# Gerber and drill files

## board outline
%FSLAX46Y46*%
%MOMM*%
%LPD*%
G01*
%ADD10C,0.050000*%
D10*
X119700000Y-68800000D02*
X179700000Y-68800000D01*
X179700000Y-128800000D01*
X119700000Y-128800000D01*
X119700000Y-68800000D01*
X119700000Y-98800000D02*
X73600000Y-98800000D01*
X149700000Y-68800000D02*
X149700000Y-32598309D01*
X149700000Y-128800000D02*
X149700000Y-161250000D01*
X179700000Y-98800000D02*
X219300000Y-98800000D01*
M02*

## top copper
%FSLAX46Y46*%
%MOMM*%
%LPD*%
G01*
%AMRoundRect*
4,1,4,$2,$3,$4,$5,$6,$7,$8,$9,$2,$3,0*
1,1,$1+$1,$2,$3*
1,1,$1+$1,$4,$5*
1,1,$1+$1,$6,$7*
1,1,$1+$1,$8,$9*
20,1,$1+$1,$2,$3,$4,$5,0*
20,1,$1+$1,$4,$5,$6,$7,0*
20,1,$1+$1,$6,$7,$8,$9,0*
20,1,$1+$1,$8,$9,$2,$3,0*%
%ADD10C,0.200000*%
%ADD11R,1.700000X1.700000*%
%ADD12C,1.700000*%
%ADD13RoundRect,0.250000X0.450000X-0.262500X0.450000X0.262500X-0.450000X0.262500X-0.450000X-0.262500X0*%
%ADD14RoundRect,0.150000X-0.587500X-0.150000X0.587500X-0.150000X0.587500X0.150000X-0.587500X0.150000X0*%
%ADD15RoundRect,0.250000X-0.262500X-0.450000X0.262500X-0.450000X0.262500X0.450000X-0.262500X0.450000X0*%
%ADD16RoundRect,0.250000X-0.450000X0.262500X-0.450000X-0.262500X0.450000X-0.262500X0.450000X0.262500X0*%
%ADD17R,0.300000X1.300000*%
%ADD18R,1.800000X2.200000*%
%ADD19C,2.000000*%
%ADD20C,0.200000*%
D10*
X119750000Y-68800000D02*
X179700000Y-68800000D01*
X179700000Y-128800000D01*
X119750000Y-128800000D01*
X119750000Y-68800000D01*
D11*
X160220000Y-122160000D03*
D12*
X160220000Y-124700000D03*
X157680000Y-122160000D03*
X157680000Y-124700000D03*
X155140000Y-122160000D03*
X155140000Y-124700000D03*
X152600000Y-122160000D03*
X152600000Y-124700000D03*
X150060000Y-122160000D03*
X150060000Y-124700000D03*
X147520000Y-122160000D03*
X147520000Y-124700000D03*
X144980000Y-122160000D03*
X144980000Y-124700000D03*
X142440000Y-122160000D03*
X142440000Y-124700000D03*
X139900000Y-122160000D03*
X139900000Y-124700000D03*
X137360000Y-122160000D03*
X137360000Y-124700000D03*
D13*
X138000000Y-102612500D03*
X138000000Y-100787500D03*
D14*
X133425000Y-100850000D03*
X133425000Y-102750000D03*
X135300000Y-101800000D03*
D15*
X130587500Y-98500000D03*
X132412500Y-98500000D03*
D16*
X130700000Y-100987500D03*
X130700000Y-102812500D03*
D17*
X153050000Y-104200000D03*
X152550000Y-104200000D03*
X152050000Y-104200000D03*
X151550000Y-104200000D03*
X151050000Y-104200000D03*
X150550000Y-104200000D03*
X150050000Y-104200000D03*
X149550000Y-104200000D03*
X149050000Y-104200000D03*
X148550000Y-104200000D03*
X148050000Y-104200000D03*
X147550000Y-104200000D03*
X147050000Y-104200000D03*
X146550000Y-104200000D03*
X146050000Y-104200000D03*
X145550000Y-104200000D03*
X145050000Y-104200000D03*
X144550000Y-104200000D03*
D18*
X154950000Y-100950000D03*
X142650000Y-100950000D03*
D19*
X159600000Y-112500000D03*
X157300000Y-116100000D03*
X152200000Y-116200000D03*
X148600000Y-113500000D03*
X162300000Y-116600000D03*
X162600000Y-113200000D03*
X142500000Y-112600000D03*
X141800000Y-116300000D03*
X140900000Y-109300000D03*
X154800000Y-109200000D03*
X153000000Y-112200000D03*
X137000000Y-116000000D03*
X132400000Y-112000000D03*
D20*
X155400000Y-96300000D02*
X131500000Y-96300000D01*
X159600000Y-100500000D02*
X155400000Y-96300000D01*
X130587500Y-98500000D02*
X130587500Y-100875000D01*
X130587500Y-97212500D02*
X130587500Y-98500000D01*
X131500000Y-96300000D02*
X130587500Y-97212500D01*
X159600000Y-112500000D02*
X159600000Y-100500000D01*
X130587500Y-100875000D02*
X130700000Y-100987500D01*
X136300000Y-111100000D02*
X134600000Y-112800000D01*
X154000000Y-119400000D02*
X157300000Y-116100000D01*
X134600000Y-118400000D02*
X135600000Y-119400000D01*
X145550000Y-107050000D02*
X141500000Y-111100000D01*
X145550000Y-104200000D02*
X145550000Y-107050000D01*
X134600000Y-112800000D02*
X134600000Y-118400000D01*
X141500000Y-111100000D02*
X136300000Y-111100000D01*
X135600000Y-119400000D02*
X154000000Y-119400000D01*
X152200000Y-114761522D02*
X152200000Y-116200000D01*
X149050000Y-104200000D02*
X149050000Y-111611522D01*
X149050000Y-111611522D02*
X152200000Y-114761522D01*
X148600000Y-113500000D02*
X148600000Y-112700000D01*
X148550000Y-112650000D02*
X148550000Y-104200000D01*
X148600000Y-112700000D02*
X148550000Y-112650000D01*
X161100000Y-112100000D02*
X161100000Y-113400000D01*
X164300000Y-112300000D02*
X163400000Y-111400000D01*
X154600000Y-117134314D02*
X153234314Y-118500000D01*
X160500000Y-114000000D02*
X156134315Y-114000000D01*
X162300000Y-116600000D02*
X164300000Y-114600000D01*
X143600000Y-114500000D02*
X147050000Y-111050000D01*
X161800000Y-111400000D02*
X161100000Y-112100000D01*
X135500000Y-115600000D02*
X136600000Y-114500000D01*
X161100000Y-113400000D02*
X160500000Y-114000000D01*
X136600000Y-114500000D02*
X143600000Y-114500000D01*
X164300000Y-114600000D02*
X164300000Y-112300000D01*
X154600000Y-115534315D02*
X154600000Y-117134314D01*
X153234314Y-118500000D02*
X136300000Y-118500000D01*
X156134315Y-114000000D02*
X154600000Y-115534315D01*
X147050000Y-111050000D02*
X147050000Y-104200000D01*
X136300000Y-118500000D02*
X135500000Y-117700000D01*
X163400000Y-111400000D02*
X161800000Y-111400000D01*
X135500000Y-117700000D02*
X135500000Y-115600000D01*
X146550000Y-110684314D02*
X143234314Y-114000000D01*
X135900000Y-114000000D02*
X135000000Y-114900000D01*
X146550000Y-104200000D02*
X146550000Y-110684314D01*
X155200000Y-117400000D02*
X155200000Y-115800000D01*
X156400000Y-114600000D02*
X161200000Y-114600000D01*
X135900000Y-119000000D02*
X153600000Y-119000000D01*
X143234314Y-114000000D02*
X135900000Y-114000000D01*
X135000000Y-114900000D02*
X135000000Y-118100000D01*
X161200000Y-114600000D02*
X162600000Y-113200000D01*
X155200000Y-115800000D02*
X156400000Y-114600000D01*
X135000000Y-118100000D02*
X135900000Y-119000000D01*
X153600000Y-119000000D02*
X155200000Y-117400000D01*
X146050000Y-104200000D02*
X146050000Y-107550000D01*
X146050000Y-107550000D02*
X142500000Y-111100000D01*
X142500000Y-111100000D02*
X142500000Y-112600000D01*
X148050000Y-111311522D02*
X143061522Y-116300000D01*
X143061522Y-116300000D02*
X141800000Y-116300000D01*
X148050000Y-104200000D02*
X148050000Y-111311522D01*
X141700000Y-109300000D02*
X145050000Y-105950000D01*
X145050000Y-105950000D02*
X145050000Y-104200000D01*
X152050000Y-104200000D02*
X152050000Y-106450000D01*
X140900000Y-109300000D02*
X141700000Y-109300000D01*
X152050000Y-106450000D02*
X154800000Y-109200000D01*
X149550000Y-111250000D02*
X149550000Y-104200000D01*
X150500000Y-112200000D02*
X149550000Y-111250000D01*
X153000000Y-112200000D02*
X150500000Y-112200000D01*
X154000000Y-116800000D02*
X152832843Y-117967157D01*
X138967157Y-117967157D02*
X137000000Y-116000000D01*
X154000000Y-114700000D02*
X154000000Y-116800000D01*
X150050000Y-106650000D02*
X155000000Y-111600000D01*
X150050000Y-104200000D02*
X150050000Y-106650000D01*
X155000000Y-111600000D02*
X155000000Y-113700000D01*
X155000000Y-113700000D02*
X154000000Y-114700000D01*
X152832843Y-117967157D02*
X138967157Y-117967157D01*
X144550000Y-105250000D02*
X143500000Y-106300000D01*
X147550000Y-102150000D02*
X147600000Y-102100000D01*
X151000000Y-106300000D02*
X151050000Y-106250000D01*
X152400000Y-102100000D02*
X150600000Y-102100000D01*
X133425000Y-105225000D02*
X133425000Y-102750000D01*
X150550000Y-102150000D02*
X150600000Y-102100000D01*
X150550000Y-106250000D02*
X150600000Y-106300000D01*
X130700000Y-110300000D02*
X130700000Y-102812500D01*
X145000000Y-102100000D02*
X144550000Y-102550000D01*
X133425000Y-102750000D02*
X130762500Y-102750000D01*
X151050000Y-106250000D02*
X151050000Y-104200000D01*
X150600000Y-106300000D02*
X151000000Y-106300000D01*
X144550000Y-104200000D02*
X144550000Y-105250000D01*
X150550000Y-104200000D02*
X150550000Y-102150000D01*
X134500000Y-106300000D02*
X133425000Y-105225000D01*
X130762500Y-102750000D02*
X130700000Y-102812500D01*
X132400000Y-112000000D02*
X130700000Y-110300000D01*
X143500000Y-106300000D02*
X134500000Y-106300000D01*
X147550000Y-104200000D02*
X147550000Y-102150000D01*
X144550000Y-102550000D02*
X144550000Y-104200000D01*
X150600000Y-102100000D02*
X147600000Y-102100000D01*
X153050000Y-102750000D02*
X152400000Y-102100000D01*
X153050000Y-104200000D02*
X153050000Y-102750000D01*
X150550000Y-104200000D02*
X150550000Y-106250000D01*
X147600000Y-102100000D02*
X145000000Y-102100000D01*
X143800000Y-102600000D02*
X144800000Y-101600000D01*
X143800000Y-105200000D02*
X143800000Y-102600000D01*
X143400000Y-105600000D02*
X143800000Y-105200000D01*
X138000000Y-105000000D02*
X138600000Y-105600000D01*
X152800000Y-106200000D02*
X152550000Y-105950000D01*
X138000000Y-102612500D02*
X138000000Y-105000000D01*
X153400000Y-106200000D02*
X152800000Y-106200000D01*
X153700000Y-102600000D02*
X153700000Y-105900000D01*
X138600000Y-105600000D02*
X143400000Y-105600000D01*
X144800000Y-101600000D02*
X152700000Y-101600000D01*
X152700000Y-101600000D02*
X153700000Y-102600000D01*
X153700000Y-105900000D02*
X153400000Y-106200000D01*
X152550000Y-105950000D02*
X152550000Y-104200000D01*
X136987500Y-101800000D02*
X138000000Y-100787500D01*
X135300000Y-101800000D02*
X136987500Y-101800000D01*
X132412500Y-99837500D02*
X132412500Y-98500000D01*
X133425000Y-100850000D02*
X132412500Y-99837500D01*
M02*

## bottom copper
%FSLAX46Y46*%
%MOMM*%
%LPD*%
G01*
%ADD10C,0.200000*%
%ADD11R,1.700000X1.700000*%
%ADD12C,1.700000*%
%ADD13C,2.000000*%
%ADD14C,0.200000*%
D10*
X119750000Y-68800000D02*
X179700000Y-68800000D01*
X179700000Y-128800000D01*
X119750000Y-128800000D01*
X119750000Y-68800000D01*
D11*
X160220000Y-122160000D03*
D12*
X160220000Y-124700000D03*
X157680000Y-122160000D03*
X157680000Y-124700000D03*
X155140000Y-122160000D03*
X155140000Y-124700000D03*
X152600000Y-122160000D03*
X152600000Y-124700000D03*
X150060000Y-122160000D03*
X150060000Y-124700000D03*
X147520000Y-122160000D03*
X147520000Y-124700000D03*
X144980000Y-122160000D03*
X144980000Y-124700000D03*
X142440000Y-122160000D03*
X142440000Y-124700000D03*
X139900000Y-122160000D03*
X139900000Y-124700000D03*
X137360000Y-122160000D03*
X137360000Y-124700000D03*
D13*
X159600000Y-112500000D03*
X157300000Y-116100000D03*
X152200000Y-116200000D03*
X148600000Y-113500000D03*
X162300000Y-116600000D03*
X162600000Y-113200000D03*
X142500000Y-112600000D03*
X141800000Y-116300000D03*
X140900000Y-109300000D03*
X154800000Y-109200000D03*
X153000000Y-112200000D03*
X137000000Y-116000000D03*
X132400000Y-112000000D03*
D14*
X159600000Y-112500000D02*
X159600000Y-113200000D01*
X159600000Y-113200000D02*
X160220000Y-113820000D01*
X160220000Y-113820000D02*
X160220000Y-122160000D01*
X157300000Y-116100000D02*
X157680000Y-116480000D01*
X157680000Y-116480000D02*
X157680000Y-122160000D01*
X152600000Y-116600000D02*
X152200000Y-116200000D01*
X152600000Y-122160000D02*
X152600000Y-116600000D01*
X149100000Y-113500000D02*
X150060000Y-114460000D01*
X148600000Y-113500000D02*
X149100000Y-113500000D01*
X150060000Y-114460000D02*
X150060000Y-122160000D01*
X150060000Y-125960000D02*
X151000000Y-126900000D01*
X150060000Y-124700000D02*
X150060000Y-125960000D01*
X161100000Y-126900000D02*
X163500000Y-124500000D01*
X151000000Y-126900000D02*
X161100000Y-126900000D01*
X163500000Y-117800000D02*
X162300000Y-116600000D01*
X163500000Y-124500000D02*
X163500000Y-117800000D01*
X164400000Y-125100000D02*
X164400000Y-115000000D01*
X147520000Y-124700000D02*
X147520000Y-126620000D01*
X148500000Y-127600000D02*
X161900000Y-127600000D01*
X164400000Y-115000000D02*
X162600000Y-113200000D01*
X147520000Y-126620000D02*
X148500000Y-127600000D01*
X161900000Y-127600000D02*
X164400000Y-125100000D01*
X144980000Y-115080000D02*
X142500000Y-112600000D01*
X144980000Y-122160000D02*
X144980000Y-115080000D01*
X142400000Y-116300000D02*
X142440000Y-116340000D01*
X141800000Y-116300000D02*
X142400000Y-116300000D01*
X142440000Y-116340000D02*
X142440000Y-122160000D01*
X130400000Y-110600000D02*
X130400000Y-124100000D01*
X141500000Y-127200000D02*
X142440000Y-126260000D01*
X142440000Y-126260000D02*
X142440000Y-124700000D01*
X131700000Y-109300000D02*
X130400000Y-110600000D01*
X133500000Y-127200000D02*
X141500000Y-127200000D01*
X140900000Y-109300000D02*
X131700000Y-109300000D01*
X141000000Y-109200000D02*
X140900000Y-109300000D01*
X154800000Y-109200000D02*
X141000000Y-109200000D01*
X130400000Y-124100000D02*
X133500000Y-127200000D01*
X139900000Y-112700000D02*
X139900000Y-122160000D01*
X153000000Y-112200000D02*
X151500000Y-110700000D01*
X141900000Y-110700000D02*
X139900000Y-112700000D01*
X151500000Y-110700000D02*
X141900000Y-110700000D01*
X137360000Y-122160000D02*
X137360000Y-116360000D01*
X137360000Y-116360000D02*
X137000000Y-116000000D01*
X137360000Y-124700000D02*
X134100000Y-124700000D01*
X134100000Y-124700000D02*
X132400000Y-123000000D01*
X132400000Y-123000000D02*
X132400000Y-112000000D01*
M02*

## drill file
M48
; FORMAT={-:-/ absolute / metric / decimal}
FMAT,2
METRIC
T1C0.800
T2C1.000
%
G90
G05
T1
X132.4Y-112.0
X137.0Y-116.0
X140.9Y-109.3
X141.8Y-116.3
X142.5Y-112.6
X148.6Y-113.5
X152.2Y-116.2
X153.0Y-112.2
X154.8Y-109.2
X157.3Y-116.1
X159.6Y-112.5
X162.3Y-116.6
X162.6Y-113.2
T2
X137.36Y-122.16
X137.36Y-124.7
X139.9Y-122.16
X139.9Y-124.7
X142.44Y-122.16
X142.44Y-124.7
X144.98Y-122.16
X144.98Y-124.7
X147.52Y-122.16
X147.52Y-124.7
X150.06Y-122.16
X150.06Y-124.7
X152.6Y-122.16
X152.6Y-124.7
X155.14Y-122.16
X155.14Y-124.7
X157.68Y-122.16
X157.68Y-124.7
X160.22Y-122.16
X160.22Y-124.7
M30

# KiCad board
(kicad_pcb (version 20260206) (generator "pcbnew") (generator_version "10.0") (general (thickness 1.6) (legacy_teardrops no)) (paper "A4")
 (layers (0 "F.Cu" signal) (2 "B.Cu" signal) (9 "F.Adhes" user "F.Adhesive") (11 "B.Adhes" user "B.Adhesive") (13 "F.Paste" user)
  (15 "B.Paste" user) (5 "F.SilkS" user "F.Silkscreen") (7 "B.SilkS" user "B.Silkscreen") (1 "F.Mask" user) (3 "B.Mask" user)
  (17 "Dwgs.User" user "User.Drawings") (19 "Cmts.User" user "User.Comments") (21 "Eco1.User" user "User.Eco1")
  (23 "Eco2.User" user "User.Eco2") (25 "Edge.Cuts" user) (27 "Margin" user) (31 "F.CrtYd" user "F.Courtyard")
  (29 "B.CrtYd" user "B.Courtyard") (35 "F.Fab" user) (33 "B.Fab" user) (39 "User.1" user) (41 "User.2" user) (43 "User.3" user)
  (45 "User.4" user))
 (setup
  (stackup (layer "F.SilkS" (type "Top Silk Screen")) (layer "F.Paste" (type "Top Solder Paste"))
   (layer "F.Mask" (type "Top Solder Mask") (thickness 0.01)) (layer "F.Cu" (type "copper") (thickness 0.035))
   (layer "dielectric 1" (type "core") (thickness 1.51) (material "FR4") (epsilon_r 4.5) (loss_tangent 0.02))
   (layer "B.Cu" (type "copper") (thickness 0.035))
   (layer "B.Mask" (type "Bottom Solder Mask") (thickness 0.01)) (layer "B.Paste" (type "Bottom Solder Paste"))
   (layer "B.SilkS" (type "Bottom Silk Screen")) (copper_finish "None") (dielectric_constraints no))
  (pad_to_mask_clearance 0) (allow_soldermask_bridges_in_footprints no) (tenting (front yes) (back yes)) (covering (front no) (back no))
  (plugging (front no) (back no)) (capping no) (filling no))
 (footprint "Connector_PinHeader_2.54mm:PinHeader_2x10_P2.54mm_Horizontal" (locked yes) (layer "F.Cu") (at 160.22 122.16 -90)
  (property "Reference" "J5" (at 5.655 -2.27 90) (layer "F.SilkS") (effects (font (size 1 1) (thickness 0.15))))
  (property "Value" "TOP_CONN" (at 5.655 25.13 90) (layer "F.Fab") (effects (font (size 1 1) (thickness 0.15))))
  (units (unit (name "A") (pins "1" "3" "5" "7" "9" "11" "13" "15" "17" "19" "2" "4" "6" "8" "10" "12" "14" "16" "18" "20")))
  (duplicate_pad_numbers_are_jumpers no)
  (pad "1" thru_hole rect (at 0 0 270) (size 1.7 1.7) (drill 1) (layers "*.Cu" "*.Mask") (remove_unused_layers no) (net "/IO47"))
  (pad "2" thru_hole circle (at 2.54 0 270) (size 1.7 1.7) (drill 1) (layers "*.Cu" "*.Mask") (remove_unused_layers no) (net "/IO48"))
  (pad "3" thru_hole circle (at 0 2.54 270) (size 1.7 1.7) (drill 1) (layers "*.Cu" "*.Mask") (remove_unused_layers no) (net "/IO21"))
  (pad "4" thru_hole circle (at 2.54 2.54 270) (size 1.7 1.7) (drill 1) (layers "*.Cu" "*.Mask") (remove_unused_layers no) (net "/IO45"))
  (pad "5" thru_hole circle (at 0 5.08 270) (size 1.7 1.7) (drill 1) (layers "*.Cu" "*.Mask") (remove_unused_layers no) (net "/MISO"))
  (pad "6" thru_hole circle (at 2.54 5.08 270) (size 1.7 1.7) (drill 1) (layers "*.Cu" "*.Mask") (remove_unused_layers no) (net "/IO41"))
  (pad "7" thru_hole circle (at 0 7.62 270) (size 1.7 1.7) (drill 1) (layers "*.Cu" "*.Mask") (remove_unused_layers no) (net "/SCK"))
  (pad "8" thru_hole circle (at 2.54 7.62 270) (size 1.7 1.7) (drill 1) (layers "*.Cu" "*.Mask") (remove_unused_layers no) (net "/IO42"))
  (pad "9" thru_hole circle (at 0 10.16 270) (size 1.7 1.7) (drill 1) (layers "*.Cu" "*.Mask") (remove_unused_layers no) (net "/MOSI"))
  (pad "10" thru_hole circle (at 2.54 10.16 270) (size 1.7 1.7) (drill 1) (layers "*.Cu" "*.Mask") (remove_unused_layers no) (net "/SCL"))
  (pad "11" thru_hole circle (at 0 12.7 270) (size 1.7 1.7) (drill 1) (layers "*.Cu" "*.Mask") (remove_unused_layers no) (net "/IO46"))
  (pad "12" thru_hole circle (at 2.54 12.7 270) (size 1.7 1.7) (drill 1) (layers "*.Cu" "*.Mask") (remove_unused_layers no) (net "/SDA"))
  (pad "13" thru_hole circle (at 0 15.24 270) (size 1.7 1.7) (drill 1) (layers "*.Cu" "*.Mask") (remove_unused_layers no) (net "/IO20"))
  (pad "14" thru_hole circle (at 2.54 15.24 270) (size 1.7 1.7) (drill 1) (layers "*.Cu" "*.Mask") (remove_unused_layers no) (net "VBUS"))
  (pad "15" thru_hole circle (at 0 17.78 270) (size 1.7 1.7) (drill 1) (layers "*.Cu" "*.Mask") (remove_unused_layers no) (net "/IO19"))
  (pad "16" thru_hole circle (at 2.54 17.78 270) (size 1.7 1.7) (drill 1) (layers "*.Cu" "*.Mask") (remove_unused_layers no) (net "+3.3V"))
  (pad "17" thru_hole circle (at 0 20.32 270) (size 1.7 1.7) (drill 1) (layers "*.Cu" "*.Mask") (remove_unused_layers no) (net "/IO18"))
  (pad "18" thru_hole circle (at 2.54 20.32 270) (size 1.7 1.7) (drill 1) (layers "*.Cu" "*.Mask") (remove_unused_layers no) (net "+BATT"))
  (pad "19" thru_hole circle (at 0 22.86 270) (size 1.7 1.7) (drill 1) (layers "*.Cu" "*.Mask") (remove_unused_layers no) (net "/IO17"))
  (pad "20" thru_hole circle (at 2.54 22.86 270) (size 1.7 1.7) (drill 1) (layers "*.Cu" "*.Mask") (remove_unused_layers no) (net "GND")))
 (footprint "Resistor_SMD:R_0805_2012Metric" (layer "F.Cu") (at 138 101.7 90)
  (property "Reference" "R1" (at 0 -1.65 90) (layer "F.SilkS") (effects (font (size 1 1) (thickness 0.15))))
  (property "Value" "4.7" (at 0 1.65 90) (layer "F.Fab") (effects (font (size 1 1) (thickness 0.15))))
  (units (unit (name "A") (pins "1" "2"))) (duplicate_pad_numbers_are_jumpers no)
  (pad "1" smd roundrect (at -0.9125 0 90) (size 1.025 1.4) (layers "F.Cu" "F.Mask" "F.Paste") (roundrect_rratio 0.243902) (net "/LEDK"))
  (pad "2" smd roundrect (at 0.9125 0 90) (size 1.025 1.4) (layers "F.Cu" "F.Mask" "F.Paste") (roundrect_rratio 0.243902) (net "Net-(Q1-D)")))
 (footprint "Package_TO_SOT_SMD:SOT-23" (layer "F.Cu") (at 134.3625 101.8)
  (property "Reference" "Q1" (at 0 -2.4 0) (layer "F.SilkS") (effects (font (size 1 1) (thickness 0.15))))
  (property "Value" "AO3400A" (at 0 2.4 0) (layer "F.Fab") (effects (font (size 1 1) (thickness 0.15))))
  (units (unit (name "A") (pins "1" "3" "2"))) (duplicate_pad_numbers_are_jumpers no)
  (pad "1" smd roundrect (at -0.9375 -0.95) (size 1.475 0.6) (layers "F.Cu" "F.Mask" "F.Paste") (roundrect_rratio 0.25) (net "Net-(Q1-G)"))
  (pad "2" smd roundrect (at -0.9375 0.95) (size 1.475 0.6) (layers "F.Cu" "F.Mask" "F.Paste") (roundrect_rratio 0.25) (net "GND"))
  (pad "3" smd roundrect (at 0.9375 0) (size 1.475 0.6) (layers "F.Cu" "F.Mask" "F.Paste") (roundrect_rratio 0.25) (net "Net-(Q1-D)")))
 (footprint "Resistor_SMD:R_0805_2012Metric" (layer "F.Cu") (at 131.5 98.5)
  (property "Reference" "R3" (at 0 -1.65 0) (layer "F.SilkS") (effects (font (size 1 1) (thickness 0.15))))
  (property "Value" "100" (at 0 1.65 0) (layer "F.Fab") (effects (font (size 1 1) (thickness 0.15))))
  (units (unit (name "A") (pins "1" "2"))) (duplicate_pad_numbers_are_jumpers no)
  (pad "1" smd roundrect (at -0.9125 0) (size 1.025 1.4) (layers "F.Cu" "F.Mask" "F.Paste") (roundrect_rratio 0.243902) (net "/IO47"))
  (pad "2" smd roundrect (at 0.9125 0) (size 1.025 1.4) (layers "F.Cu" "F.Mask" "F.Paste") (roundrect_rratio 0.243902) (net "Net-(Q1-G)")))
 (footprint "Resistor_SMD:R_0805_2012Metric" (layer "F.Cu") (at 130.7 101.9 -90)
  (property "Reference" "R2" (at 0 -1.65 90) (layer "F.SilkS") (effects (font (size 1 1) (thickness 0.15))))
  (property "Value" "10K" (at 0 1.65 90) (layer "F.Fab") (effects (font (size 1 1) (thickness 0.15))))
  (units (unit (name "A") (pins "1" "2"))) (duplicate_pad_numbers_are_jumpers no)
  (pad "1" smd roundrect (at -0.9125 0 270) (size 1.025 1.4) (layers "F.Cu" "F.Mask" "F.Paste") (roundrect_rratio 0.243902) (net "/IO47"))
  (pad "2" smd roundrect (at 0.9125 0 270) (size 1.025 1.4) (layers "F.Cu" "F.Mask" "F.Paste") (roundrect_rratio 0.243902) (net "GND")))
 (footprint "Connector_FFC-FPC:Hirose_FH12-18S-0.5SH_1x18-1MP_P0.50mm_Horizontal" (layer "F.Cu") (at 148.8 102.35 180)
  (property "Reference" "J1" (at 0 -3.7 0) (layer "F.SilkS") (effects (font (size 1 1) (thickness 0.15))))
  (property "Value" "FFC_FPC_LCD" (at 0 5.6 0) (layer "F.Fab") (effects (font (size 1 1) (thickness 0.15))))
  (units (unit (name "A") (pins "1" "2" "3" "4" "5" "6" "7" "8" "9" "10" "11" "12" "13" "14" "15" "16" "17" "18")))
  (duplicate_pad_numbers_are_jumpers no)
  (pad "1" smd rect (at -4.25 -1.85 180) (size 0.3 1.3) (layers "F.Cu" "F.Mask" "F.Paste") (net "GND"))
  (pad "2" smd rect (at -3.75 -1.85 180) (size 0.3 1.3) (layers "F.Cu" "F.Mask" "F.Paste") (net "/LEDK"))
  (pad "3" smd rect (at -3.25 -1.85 180) (size 0.3 1.3) (layers "F.Cu" "F.Mask" "F.Paste") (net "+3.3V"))
  (pad "4" smd rect (at -2.75 -1.85 180) (size 0.3 1.3) (layers "F.Cu" "F.Mask" "F.Paste") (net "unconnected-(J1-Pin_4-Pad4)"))
  (pad "5" smd rect (at -2.25 -1.85 180) (size 0.3 1.3) (layers "F.Cu" "F.Mask" "F.Paste") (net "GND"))
  (pad "6" smd rect (at -1.75 -1.85 180) (size 0.3 1.3) (layers "F.Cu" "F.Mask" "F.Paste") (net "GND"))
  (pad "7" smd rect (at -1.25 -1.85 180) (size 0.3 1.3) (layers "F.Cu" "F.Mask" "F.Paste") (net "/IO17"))
  (pad "8" smd rect (at -0.75 -1.85 180) (size 0.3 1.3) (layers "F.Cu" "F.Mask" "F.Paste") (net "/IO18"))
  (pad "9" smd rect (at -0.25 -1.85 180) (size 0.3 1.3) (layers "F.Cu" "F.Mask" "F.Paste") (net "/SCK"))
  (pad "10" smd rect (at 0.25 -1.85 180) (size 0.3 1.3) (layers "F.Cu" "F.Mask" "F.Paste") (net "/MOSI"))
  (pad "11" smd rect (at 0.75 -1.85 180) (size 0.3 1.3) (layers "F.Cu" "F.Mask" "F.Paste") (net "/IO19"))
  (pad "12" smd rect (at 1.25 -1.85 180) (size 0.3 1.3) (layers "F.Cu" "F.Mask" "F.Paste") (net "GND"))
  (pad "13" smd rect (at 1.75 -1.85 180) (size 0.3 1.3) (layers "F.Cu" "F.Mask" "F.Paste") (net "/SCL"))
  (pad "14" smd rect (at 2.25 -1.85 180) (size 0.3 1.3) (layers "F.Cu" "F.Mask" "F.Paste") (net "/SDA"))
  (pad "15" smd rect (at 2.75 -1.85 180) (size 0.3 1.3) (layers "F.Cu" "F.Mask" "F.Paste") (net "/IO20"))
  (pad "16" smd rect (at 3.25 -1.85 180) (size 0.3 1.3) (layers "F.Cu" "F.Mask" "F.Paste") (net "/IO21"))
  (pad "17" smd rect (at 3.75 -1.85 180) (size 0.3 1.3) (layers "F.Cu" "F.Mask" "F.Paste") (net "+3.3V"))
  (pad "18" smd rect (at 4.25 -1.85 180) (size 0.3 1.3) (layers "F.Cu" "F.Mask" "F.Paste") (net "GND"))
  (pad "MP" smd rect (at -6.15 1.4 180) (size 1.8 2.2) (layers "F.Cu" "F.Mask" "F.Paste"))
  (pad "MP" smd rect (at 6.15 1.4 180) (size 1.8 2.2) (layers "F.Cu" "F.Mask" "F.Paste")))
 (gr_rect (start 119.75 68.8) (end 179.7 128.8) (stroke (width 0.2) (type default)) (fill no) (layer "F.Cu"))
 (gr_rect (start 119.75 68.8) (end 179.7 128.8) (stroke (width 0.2) (type default)) (fill no) (layer "B.Cu"))
 (gr_rect (start 119.7 68.8) (end 179.7 128.8) (stroke (width 0.05) (type solid)) (fill no) (layer "Edge.Cuts"))
 (gr_line (start 119.7 98.8) (end 73.6 98.8) (stroke (width 0.05) (type default)) (layer "Edge.Cuts"))
 (gr_line (start 149.7 68.8) (end 149.7 32.598309) (stroke (width 0.05) (type solid)) (layer "Edge.Cuts"))
 (gr_line (start 149.7 128.8) (end 149.7 161.25) (stroke (width 0.05) (type default)) (layer "Edge.Cuts"))
 (gr_line (start 179.7 98.8) (end 219.3 98.8) (stroke (width 0.05) (type default)) (layer "Edge.Cuts"))
 (segment (start 155.4 96.3) (end 131.5 96.3) (width 0.2) (layer "F.Cu") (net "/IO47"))
 (segment (start 159.6 100.5) (end 155.4 96.3) (width 0.2) (layer "F.Cu") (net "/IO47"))
 (segment (start 130.5875 98.5) (end 130.5875 100.875) (width 0.2) (layer "F.Cu") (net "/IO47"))
 (segment (start 130.5875 97.2125) (end 130.5875 98.5) (width 0.2) (layer "F.Cu") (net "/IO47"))
 (segment (start 131.5 96.3) (end 130.5875 97.2125) (width 0.2) (layer "F.Cu") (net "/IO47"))
 (segment (start 159.6 112.5) (end 159.6 100.5) (width 0.2) (layer "F.Cu") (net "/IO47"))
 (segment (start 130.5875 100.875) (end 130.7 100.9875) (width 0.2) (layer "F.Cu") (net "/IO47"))
 (via (at 159.6 112.5) (size 2) (drill 0.8) (layers "F.Cu" "B.Cu") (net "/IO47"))
 (segment (start 159.6 112.5) (end 159.6 113.2) (width 0.2) (layer "B.Cu") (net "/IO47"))
 (segment (start 159.6 113.2) (end 160.22 113.82) (width 0.2) (layer "B.Cu") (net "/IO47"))
 (segment (start 160.22 113.82) (end 160.22 122.16) (width 0.2) (layer "B.Cu") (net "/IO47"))
 (segment (start 136.3 111.1) (end 134.6 112.8) (width 0.2) (layer "F.Cu") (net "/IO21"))
 (segment (start 154 119.4) (end 157.3 116.1) (width 0.2) (layer "F.Cu") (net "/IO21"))
 (segment (start 134.6 118.4) (end 135.6 119.4) (width 0.2) (layer "F.Cu") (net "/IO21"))
 (segment (start 145.55 107.05) (end 141.5 111.1) (width 0.2) (layer "F.Cu") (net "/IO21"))
 (segment (start 145.55 104.2) (end 145.55 107.05) (width 0.2) (layer "F.Cu") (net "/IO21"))
 (segment (start 134.6 112.8) (end 134.6 118.4) (width 0.2) (layer "F.Cu") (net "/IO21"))
 (segment (start 141.5 111.1) (end 136.3 111.1) (width 0.2) (layer "F.Cu") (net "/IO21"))
 (segment (start 135.6 119.4) (end 154 119.4) (width 0.2) (layer "F.Cu") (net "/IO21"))
 (via (at 157.3 116.1) (size 2) (drill 0.8) (layers "F.Cu" "B.Cu") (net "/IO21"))
 (segment (start 157.3 116.1) (end 157.68 116.48) (width 0.2) (layer "B.Cu") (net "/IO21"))
 (segment (start 157.68 116.48) (end 157.68 122.16) (width 0.2) (layer "B.Cu") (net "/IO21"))
 (segment (start 152.2 114.761522) (end 152.2 116.2) (width 0.2) (layer "F.Cu") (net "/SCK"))
 (segment (start 149.05 104.2) (end 149.05 111.611522) (width 0.2) (layer "F.Cu") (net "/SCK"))
 (segment (start 149.05 111.611522) (end 152.2 114.761522) (width 0.2) (layer "F.Cu") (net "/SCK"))
 (via (at 152.2 116.2) (size 2) (drill 0.8) (layers "F.Cu" "B.Cu") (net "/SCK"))
 (segment (start 152.6 116.6) (end 152.2 116.2) (width 0.2) (layer "B.Cu") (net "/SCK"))
 (segment (start 152.6 122.16) (end 152.6 116.6) (width 0.2) (layer "B.Cu") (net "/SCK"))
 (segment (start 148.6 113.5) (end 148.6 112.7) (width 0.2) (layer "F.Cu") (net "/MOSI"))
 (segment (start 148.55 112.65) (end 148.55 104.2) (width 0.2) (layer "F.Cu") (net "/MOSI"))
 (segment (start 148.6 112.7) (end 148.55 112.65) (width 0.2) (layer "F.Cu") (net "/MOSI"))
 (via (at 148.6 113.5) (size 2) (drill 0.8) (layers "F.Cu" "B.Cu") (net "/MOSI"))
 (segment (start 149.1 113.5) (end 150.06 114.46) (width 0.2) (layer "B.Cu") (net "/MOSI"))
 (segment (start 148.6 113.5) (end 149.1 113.5) (width 0.2) (layer "B.Cu") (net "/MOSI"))
 (segment (start 150.06 114.46) (end 150.06 122.16) (width 0.2) (layer "B.Cu") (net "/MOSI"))
 (segment (start 161.1 112.1) (end 161.1 113.4) (width 0.2) (layer "F.Cu") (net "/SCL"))
 (segment (start 164.3 112.3) (end 163.4 111.4) (width 0.2) (layer "F.Cu") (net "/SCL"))
 (segment (start 154.6 117.134314) (end 153.234314 118.5) (width 0.2) (layer "F.Cu") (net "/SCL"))
 (segment (start 160.5 114) (end 156.134315 114) (width 0.2) (layer "F.Cu") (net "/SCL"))
 (segment (start 162.3 116.6) (end 164.3 114.6) (width 0.2) (layer "F.Cu") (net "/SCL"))
 (segment (start 143.6 114.5) (end 147.05 111.05) (width 0.2) (layer "F.Cu") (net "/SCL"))
 (segment (start 161.8 111.4) (end 161.1 112.1) (width 0.2) (layer "F.Cu") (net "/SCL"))
 (segment (start 135.5 115.6) (end 136.6 114.5) (width 0.2) (layer "F.Cu") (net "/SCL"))
 (segment (start 161.1 113.4) (end 160.5 114) (width 0.2) (layer "F.Cu") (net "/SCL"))
 (segment (start 136.6 114.5) (end 143.6 114.5) (width 0.2) (layer "F.Cu") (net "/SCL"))
 (segment (start 164.3 114.6) (end 164.3 112.3) (width 0.2) (layer "F.Cu") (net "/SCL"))
 (segment (start 154.6 115.534315) (end 154.6 117.134314) (width 0.2) (layer "F.Cu") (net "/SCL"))
 (segment (start 153.234314 118.5) (end 136.3 118.5) (width 0.2) (layer "F.Cu") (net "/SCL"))
 (segment (start 156.134315 114) (end 154.6 115.534315) (width 0.2) (layer "F.Cu") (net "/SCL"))
 (segment (start 147.05 111.05) (end 147.05 104.2) (width 0.2) (layer "F.Cu") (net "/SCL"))
 (segment (start 136.3 118.5) (end 135.5 117.7) (width 0.2) (layer "F.Cu") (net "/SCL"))
 (segment (start 163.4 111.4) (end 161.8 111.4) (width 0.2) (layer "F.Cu") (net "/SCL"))
 (segment (start 135.5 117.7) (end 135.5 115.6) (width 0.2) (layer "F.Cu") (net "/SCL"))
 (via (at 162.3 116.6) (size 2) (drill 0.8) (layers "F.Cu" "B.Cu") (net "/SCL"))
 (segment (start 150.06 125.96) (end 151 126.9) (width 0.2) (layer "B.Cu") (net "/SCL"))
 (segment (start 150.06 124.7) (end 150.06 125.96) (width 0.2) (layer "B.Cu") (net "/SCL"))
 (segment (start 161.1 126.9) (end 163.5 124.5) (width 0.2) (layer "B.Cu") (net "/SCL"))
 (segment (start 151 126.9) (end 161.1 126.9) (width 0.2) (layer "B.Cu") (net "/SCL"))
 (segment (start 163.5 117.8) (end 162.3 116.6) (width 0.2) (layer "B.Cu") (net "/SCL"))
 (segment (start 163.5 124.5) (end 163.5 117.8) (width 0.2) (layer "B.Cu") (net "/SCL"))
 (segment (start 146.55 110.684314) (end 143.234314 114) (width 0.2) (layer "F.Cu") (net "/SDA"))
 (segment (start 135.9 114) (end 135 114.9) (width 0.2) (layer "F.Cu") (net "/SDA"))
 (segment (start 146.55 104.2) (end 146.55 110.684314) (width 0.2) (layer "F.Cu") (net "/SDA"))
 (segment (start 155.2 117.4) (end 155.2 115.8) (width 0.2) (layer "F.Cu") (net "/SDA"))
 (segment (start 156.4 114.6) (end 161.2 114.6) (width 0.2) (layer "F.Cu") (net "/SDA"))
 (segment (start 135.9 119) (end 153.6 119) (width 0.2) (layer "F.Cu") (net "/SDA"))
 (segment (start 143.234314 114) (end 135.9 114) (width 0.2) (layer "F.Cu") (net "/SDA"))
 (segment (start 135 114.9) (end 135 118.1) (width 0.2) (layer "F.Cu") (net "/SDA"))
 (segment (start 161.2 114.6) (end 162.6 113.2) (width 0.2) (layer "F.Cu") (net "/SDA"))
 (segment (start 155.2 115.8) (end 156.4 114.6) (width 0.2) (layer "F.Cu") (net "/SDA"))
 (segment (start 135 118.1) (end 135.9 119) (width 0.2) (layer "F.Cu") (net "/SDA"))
 (segment (start 153.6 119) (end 155.2 117.4) (width 0.2) (layer "F.Cu") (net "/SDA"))
 (via (at 162.6 113.2) (size 2) (drill 0.8) (layers "F.Cu" "B.Cu") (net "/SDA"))
 (segment (start 164.4 125.1) (end 164.4 115) (width 0.2) (layer "B.Cu") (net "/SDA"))
 (segment (start 147.52 124.7) (end 147.52 126.62) (width 0.2) (layer "B.Cu") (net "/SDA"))
 (segment (start 148.5 127.6) (end 161.9 127.6) (width 0.2) (layer "B.Cu") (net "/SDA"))
 (segment (start 164.4 115) (end 162.6 113.2) (width 0.2) (layer "B.Cu") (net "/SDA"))
 (segment (start 147.52 126.62) (end 148.5 127.6) (width 0.2) (layer "B.Cu") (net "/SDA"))
 (segment (start 161.9 127.6) (end 164.4 125.1) (width 0.2) (layer "B.Cu") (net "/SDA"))
 (segment (start 146.05 104.2) (end 146.05 107.55) (width 0.2) (layer "F.Cu") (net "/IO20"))
 (segment (start 146.05 107.55) (end 142.5 111.1) (width 0.2) (layer "F.Cu") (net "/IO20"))
 (segment (start 142.5 111.1) (end 142.5 112.6) (width 0.2) (layer "F.Cu") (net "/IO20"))
 (via (at 142.5 112.6) (size 2) (drill 0.8) (layers "F.Cu" "B.Cu") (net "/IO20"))
 (segment (start 144.98 115.08) (end 142.5 112.6) (width 0.2) (layer "B.Cu") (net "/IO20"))
 (segment (start 144.98 122.16) (end 144.98 115.08) (width 0.2) (layer "B.Cu") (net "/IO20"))
 (segment (start 148.05 111.311522) (end 143.061522 116.3) (width 0.2) (layer "F.Cu") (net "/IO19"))
 (segment (start 143.061522 116.3) (end 141.8 116.3) (width 0.2) (layer "F.Cu") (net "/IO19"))
 (segment (start 148.05 104.2) (end 148.05 111.311522) (width 0.2) (layer "F.Cu") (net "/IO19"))
 (via (at 141.8 116.3) (size 2) (drill 0.8) (layers "F.Cu" "B.Cu") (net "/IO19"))
 (segment (start 142.4 116.3) (end 142.44 116.34) (width 0.2) (layer "B.Cu") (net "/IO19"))
 (segment (start 141.8 116.3) (end 142.4 116.3) (width 0.2) (layer "B.Cu") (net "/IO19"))
 (segment (start 142.44 116.34) (end 142.44 122.16) (width 0.2) (layer "B.Cu") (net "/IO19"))
 (segment (start 141.7 109.3) (end 145.05 105.95) (width 0.2) (layer "F.Cu") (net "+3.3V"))
 (segment (start 145.05 105.95) (end 145.05 104.2) (width 0.2) (layer "F.Cu") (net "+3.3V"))
 (segment (start 152.05 104.2) (end 152.05 106.45) (width 0.2) (layer "F.Cu") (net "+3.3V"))
 (segment (start 140.9 109.3) (end 141.7 109.3) (width 0.2) (layer "F.Cu") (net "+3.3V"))
 (segment (start 152.05 106.45) (end 154.8 109.2) (width 0.2) (layer "F.Cu") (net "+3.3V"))
 (via (at 140.9 109.3) (size 2) (drill 0.8) (layers "F.Cu" "B.Cu") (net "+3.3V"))
 (via (at 154.8 109.2) (size 2) (drill 0.8) (layers "F.Cu" "B.Cu") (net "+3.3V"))
 (segment (start 130.4 110.6) (end 130.4 124.1) (width 0.2) (layer "B.Cu") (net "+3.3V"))
 (segment (start 141.5 127.2) (end 142.44 126.26) (width 0.2) (layer "B.Cu") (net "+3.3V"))
 (segment (start 142.44 126.26) (end 142.44 124.7) (width 0.2) (layer "B.Cu") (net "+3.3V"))
 (segment (start 131.7 109.3) (end 130.4 110.6) (width 0.2) (layer "B.Cu") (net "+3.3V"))
 (segment (start 133.5 127.2) (end 141.5 127.2) (width 0.2) (layer "B.Cu") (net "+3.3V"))
 (segment (start 140.9 109.3) (end 131.7 109.3) (width 0.2) (layer "B.Cu") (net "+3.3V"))
 (segment (start 141 109.2) (end 140.9 109.3) (width 0.2) (layer "B.Cu") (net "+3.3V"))
 (segment (start 154.8 109.2) (end 141 109.2) (width 0.2) (layer "B.Cu") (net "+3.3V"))
 (segment (start 130.4 124.1) (end 133.5 127.2) (width 0.2) (layer "B.Cu") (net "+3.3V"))
 (segment (start 149.55 111.25) (end 149.55 104.2) (width 0.2) (layer "F.Cu") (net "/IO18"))
 (segment (start 150.5 112.2) (end 149.55 111.25) (width 0.2) (layer "F.Cu") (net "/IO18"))
 (segment (start 153 112.2) (end 150.5 112.2) (width 0.2) (layer "F.Cu") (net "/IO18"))
 (via (at 153 112.2) (size 2) (drill 0.8) (layers "F.Cu" "B.Cu") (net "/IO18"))
 (segment (start 139.9 112.7) (end 139.9 122.16) (width 0.2) (layer "B.Cu") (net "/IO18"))
 (segment (start 153 112.2) (end 151.5 110.7) (width 0.2) (layer "B.Cu") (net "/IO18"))
 (segment (start 141.9 110.7) (end 139.9 112.7) (width 0.2) (layer "B.Cu") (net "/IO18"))
 (segment (start 151.5 110.7) (end 141.9 110.7) (width 0.2) (layer "B.Cu") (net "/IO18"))
 (segment (start 154 116.8) (end 152.832843 117.967157) (width 0.2) (layer "F.Cu") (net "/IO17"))
 (segment (start 138.967157 117.967157) (end 137 116) (width 0.2) (layer "F.Cu") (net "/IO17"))
 (segment (start 154 114.7) (end 154 116.8) (width 0.2) (layer "F.Cu") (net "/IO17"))
 (segment (start 150.05 106.65) (end 155 111.6) (width 0.2) (layer "F.Cu") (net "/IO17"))
 (segment (start 150.05 104.2) (end 150.05 106.65) (width 0.2) (layer "F.Cu") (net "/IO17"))
 (segment (start 155 111.6) (end 155 113.7) (width 0.2) (layer "F.Cu") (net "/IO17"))
 (segment (start 155 113.7) (end 154 114.7) (width 0.2) (layer "F.Cu") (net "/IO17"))
 (segment (start 152.832843 117.967157) (end 138.967157 117.967157) (width 0.2) (layer "F.Cu") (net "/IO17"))
 (via (at 137 116) (size 2) (drill 0.8) (layers "F.Cu" "B.Cu") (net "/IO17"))
 (segment (start 137.36 122.16) (end 137.36 116.36) (width 0.2) (layer "B.Cu") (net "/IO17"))
 (segment (start 137.36 116.36) (end 137 116) (width 0.2) (layer "B.Cu") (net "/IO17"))
 (segment (start 144.55 105.25) (end 143.5 106.3) (width 0.2) (layer "F.Cu") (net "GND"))
 (segment (start 147.55 102.15) (end 147.6 102.1) (width 0.2) (layer "F.Cu") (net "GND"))
 (segment (start 151 106.3) (end 151.05 106.25) (width 0.2) (layer "F.Cu") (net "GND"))
 (segment (start 152.4 102.1) (end 150.6 102.1) (width 0.2) (layer "F.Cu") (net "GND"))
 (segment (start 133.425 105.225) (end 133.425 102.75) (width 0.2) (layer "F.Cu") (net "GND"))
 (segment (start 150.55 102.15) (end 150.6 102.1) (width 0.2) (layer "F.Cu") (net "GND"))
 (segment (start 150.55 106.25) (end 150.6 106.3) (width 0.2) (layer "F.Cu") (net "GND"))
 (segment (start 130.7 110.3) (end 130.7 102.8125) (width 0.2) (layer "F.Cu") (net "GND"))
 (segment (start 145 102.1) (end 144.55 102.55) (width 0.2) (layer "F.Cu") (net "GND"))
 (segment (start 133.425 102.75) (end 130.7625 102.75) (width 0.2) (layer "F.Cu") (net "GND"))
 (segment (start 151.05 106.25) (end 151.05 104.2) (width 0.2) (layer "F.Cu") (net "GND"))
 (segment (start 150.6 106.3) (end 151 106.3) (width 0.2) (layer "F.Cu") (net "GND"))
 (segment (start 144.55 104.2) (end 144.55 105.25) (width 0.2) (layer "F.Cu") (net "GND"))
 (segment (start 150.55 104.2) (end 150.55 102.15) (width 0.2) (layer "F.Cu") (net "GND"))
 (segment (start 134.5 106.3) (end 133.425 105.225) (width 0.2) (layer "F.Cu") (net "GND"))
 (segment (start 130.7625 102.75) (end 130.7 102.8125) (width 0.2) (layer "F.Cu") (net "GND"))
 (segment (start 132.4 112) (end 130.7 110.3) (width 0.2) (layer "F.Cu") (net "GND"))
 (segment (start 143.5 106.3) (end 134.5 106.3) (width 0.2) (layer "F.Cu") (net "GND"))
 (segment (start 147.55 104.2) (end 147.55 102.15) (width 0.2) (layer "F.Cu") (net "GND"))
 (segment (start 144.55 102.55) (end 144.55 104.2) (width 0.2) (layer "F.Cu") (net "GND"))
 (segment (start 150.6 102.1) (end 147.6 102.1) (width 0.2) (layer "F.Cu") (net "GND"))
 (segment (start 153.05 102.75) (end 152.4 102.1) (width 0.2) (layer "F.Cu") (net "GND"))
 (segment (start 153.05 104.2) (end 153.05 102.75) (width 0.2) (layer "F.Cu") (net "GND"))
 (segment (start 150.55 104.2) (end 150.55 106.25) (width 0.2) (layer "F.Cu") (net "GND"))
 (segment (start 147.6 102.1) (end 145 102.1) (width 0.2) (layer "F.Cu") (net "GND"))
 (via (at 132.4 112) (size 2) (drill 0.8) (layers "F.Cu" "B.Cu") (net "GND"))
 (segment (start 137.36 124.7) (end 134.1 124.7) (width 0.2) (layer "B.Cu") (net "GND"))
 (segment (start 134.1 124.7) (end 132.4 123) (width 0.2) (layer "B.Cu") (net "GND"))
 (segment (start 132.4 123) (end 132.4 112) (width 0.2) (layer "B.Cu") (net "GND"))
 (segment (start 143.8 102.6) (end 144.8 101.6) (width 0.2) (layer "F.Cu") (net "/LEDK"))
 (segment (start 143.8 105.2) (end 143.8 102.6) (width 0.2) (layer "F.Cu") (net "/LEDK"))
 (segment (start 143.4 105.6) (end 143.8 105.2) (width 0.2) (layer "F.Cu") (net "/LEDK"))
 (segment (start 138 105) (end 138.6 105.6) (width 0.2) (layer "F.Cu") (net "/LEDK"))
 (segment (start 152.8 106.2) (end 152.55 105.95) (width 0.2) (layer "F.Cu") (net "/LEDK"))
 (segment (start 138 102.6125) (end 138 105) (width 0.2) (layer "F.Cu") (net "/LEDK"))
 (segment (start 153.4 106.2) (end 152.8 106.2) (width 0.2) (layer "F.Cu") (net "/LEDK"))
 (segment (start 153.7 102.6) (end 153.7 105.9) (width 0.2) (layer "F.Cu") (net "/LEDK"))
 (segment (start 138.6 105.6) (end 143.4 105.6) (width 0.2) (layer "F.Cu") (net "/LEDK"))
 (segment (start 144.8 101.6) (end 152.7 101.6) (width 0.2) (layer "F.Cu") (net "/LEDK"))
 (segment (start 152.7 101.6) (end 153.7 102.6) (width 0.2) (layer "F.Cu") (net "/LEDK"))
 (segment (start 153.7 105.9) (end 153.4 106.2) (width 0.2) (layer "F.Cu") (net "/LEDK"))
 (segment (start 152.55 105.95) (end 152.55 104.2) (width 0.2) (layer "F.Cu") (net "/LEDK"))
 (segment (start 136.9875 101.8) (end 138 100.7875) (width 0.2) (layer "F.Cu") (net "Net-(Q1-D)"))
 (segment (start 135.3 101.8) (end 136.9875 101.8) (width 0.2) (layer "F.Cu") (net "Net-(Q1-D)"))
 (segment (start 132.4125 99.8375) (end 132.4125 98.5) (width 0.2) (layer "F.Cu") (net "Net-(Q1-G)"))
 (segment (start 133.425 100.85) (end 132.4125 99.8375) (width 0.2) (layer "F.Cu") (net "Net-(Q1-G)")))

